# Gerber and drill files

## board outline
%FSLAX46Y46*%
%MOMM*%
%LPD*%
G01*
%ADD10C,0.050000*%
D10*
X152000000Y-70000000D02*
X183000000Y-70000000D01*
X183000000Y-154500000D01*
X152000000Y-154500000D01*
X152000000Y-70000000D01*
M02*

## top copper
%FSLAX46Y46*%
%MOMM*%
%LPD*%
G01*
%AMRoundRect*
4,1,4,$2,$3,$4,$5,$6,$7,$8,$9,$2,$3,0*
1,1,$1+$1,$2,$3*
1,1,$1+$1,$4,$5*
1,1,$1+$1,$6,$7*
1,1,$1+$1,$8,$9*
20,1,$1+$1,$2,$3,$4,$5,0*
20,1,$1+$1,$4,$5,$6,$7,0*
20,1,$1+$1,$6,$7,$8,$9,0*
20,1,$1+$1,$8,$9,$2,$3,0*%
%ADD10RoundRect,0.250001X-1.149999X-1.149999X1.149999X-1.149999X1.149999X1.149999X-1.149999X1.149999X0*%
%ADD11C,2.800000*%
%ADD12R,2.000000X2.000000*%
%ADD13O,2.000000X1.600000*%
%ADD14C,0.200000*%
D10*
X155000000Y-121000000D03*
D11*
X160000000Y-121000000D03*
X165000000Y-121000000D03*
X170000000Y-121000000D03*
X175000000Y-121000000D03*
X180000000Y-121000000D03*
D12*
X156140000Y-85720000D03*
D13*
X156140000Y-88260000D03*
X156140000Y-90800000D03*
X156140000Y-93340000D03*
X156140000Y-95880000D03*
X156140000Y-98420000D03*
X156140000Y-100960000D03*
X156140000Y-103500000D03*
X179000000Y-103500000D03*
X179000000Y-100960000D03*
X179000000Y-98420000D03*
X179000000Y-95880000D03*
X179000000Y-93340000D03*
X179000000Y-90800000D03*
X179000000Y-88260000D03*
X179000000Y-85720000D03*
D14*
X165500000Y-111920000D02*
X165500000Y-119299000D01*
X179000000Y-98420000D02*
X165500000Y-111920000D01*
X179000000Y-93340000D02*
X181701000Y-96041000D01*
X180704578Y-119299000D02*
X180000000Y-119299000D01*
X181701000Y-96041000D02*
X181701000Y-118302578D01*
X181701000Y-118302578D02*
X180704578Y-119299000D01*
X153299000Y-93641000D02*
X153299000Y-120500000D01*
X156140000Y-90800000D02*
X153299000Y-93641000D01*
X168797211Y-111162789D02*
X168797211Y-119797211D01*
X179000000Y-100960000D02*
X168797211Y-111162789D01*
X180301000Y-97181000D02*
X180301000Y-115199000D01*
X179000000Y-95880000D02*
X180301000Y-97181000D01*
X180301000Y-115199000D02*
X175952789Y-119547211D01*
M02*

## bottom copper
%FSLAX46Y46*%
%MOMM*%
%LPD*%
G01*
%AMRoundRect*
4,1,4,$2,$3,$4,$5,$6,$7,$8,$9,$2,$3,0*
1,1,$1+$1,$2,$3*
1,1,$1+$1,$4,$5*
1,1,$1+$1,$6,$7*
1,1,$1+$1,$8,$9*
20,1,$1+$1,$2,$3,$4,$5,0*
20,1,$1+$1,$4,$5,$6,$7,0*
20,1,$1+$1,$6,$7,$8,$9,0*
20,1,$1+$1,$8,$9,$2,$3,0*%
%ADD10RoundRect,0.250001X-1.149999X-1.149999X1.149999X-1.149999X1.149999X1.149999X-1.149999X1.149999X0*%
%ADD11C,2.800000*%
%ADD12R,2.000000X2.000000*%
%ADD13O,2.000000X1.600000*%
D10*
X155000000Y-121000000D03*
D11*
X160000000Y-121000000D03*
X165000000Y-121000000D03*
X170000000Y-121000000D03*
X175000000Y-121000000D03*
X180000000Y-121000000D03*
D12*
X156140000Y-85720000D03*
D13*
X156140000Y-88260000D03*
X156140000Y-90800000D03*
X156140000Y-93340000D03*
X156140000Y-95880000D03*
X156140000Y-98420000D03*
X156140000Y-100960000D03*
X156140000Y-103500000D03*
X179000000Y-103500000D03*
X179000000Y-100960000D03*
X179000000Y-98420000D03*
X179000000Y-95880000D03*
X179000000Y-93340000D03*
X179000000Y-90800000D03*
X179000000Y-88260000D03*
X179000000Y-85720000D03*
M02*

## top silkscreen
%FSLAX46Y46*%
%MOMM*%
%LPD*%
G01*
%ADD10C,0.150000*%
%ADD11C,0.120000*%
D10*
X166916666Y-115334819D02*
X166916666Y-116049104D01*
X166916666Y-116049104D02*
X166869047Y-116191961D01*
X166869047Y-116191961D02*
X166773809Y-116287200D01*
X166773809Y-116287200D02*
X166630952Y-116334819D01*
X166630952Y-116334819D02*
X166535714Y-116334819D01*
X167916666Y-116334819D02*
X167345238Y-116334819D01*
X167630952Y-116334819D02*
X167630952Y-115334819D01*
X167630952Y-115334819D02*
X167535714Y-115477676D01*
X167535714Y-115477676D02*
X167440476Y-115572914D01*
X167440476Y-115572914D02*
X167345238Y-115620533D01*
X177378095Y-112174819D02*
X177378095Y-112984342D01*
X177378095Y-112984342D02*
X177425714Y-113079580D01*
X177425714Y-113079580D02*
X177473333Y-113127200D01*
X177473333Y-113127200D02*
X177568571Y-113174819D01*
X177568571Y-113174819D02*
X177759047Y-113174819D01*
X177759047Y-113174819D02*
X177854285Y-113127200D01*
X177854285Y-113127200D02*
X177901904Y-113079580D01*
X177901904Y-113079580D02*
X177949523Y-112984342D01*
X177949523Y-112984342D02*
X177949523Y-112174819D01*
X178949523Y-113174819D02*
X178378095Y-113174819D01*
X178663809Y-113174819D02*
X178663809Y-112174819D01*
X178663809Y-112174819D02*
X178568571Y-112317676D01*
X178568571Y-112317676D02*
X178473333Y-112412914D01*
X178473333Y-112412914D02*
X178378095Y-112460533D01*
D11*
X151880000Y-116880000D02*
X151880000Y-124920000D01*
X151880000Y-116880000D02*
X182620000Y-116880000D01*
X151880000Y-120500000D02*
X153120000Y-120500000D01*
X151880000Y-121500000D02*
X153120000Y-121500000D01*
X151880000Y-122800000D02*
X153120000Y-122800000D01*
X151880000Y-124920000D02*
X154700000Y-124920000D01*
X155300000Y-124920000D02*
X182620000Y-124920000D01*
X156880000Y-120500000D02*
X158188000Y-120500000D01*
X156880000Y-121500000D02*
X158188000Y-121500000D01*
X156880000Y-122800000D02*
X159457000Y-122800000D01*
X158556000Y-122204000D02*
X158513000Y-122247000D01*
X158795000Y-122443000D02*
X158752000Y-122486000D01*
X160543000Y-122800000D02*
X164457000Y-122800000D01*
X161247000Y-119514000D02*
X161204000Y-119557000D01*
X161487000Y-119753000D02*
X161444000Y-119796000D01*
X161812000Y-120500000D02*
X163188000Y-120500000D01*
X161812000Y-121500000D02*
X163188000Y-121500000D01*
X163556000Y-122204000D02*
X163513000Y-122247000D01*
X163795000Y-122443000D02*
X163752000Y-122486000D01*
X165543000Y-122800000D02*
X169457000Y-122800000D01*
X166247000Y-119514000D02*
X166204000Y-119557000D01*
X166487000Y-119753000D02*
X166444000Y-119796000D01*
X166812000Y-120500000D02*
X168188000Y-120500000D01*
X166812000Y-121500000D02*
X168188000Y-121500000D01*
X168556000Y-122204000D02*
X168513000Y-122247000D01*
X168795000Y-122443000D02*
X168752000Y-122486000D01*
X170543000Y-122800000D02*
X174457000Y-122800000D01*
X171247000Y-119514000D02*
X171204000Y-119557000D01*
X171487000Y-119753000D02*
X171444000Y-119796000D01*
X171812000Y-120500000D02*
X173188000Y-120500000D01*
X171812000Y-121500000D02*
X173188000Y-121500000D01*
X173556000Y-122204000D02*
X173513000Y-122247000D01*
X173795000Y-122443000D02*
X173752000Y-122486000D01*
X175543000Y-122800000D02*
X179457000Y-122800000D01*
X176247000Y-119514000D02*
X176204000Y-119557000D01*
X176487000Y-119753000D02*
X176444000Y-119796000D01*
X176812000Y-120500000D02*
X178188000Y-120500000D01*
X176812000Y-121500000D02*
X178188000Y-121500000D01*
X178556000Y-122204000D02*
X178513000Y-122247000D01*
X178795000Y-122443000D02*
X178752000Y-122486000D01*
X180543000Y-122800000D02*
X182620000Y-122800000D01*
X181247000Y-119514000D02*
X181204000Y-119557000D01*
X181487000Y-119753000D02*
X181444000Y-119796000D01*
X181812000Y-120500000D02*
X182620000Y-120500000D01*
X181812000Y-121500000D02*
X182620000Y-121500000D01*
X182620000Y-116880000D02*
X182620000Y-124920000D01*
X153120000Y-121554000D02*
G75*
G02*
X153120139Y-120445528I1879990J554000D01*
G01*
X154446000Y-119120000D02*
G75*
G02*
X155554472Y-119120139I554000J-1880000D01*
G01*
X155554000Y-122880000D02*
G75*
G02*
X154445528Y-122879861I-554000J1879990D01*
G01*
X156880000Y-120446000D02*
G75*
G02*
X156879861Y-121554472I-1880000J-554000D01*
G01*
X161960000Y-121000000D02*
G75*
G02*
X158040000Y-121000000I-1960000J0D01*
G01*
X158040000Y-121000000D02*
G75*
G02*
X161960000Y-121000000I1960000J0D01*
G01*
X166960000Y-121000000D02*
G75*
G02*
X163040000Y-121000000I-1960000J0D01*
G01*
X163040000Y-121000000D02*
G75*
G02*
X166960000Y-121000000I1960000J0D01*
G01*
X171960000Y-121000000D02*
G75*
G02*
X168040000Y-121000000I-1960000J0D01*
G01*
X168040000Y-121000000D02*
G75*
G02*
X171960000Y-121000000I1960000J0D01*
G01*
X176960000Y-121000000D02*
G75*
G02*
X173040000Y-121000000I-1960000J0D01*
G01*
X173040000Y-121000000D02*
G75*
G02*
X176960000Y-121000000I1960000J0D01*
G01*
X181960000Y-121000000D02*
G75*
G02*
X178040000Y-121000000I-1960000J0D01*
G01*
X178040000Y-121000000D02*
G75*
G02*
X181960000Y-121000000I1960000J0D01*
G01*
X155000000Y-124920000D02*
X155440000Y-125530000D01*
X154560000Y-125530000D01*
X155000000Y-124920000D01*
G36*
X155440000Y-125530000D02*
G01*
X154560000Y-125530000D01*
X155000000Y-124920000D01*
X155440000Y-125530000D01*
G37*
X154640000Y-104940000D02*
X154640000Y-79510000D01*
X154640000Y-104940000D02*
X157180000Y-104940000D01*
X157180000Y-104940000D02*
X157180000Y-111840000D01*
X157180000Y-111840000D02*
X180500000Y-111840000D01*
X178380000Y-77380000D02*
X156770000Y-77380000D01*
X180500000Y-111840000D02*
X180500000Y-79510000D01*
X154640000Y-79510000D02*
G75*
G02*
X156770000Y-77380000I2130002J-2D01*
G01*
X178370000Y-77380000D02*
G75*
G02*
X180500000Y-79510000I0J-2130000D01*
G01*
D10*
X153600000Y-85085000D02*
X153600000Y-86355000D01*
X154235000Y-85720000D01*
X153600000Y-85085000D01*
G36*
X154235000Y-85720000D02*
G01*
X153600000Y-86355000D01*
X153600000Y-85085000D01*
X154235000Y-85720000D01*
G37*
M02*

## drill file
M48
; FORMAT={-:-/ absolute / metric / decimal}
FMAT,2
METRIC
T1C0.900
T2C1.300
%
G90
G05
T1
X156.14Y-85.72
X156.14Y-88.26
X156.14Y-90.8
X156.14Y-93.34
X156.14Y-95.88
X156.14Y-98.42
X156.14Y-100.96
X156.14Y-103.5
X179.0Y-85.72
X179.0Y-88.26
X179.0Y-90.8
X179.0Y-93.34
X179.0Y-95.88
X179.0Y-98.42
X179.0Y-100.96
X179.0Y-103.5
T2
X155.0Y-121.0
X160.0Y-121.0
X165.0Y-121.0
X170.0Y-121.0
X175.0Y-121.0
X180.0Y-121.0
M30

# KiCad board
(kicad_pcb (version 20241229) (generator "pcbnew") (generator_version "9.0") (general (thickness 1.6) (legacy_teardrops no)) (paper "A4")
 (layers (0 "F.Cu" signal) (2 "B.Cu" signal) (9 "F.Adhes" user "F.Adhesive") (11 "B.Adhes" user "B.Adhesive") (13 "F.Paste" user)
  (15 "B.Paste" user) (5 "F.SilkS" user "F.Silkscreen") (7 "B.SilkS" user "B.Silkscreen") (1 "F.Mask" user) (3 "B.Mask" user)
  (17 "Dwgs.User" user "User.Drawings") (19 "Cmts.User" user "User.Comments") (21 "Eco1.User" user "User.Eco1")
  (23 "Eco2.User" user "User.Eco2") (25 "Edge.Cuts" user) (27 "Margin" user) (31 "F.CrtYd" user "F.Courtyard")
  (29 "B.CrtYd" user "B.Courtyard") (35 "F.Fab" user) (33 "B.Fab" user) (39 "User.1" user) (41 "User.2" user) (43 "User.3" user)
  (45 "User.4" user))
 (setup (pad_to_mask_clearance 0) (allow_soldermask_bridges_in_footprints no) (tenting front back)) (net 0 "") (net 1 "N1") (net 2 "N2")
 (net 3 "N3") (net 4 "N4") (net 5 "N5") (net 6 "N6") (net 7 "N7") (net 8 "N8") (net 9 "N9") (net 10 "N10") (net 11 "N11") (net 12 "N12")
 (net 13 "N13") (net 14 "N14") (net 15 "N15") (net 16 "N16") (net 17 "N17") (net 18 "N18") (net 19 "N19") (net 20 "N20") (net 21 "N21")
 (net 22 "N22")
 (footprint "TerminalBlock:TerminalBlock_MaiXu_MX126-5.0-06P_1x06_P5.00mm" (layer "F.Cu") (at 155 121)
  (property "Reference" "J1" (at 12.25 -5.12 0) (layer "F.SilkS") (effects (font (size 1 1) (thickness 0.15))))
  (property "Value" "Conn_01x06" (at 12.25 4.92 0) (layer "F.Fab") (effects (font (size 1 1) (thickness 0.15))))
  (fp_line (start -3.12 -4.12) (end -3.12 3.92) (stroke (width 0.12) (type solid)) (layer "F.SilkS"))
  (fp_line (start -3.12 -4.12) (end 27.62 -4.12) (stroke (width 0.12) (type solid)) (layer "F.SilkS"))
  (fp_line (start -3.12 -0.5) (end -1.88 -0.5) (stroke (width 0.12) (type solid)) (layer "F.SilkS"))
  (fp_line (start -3.12 0.5) (end -1.88 0.5) (stroke (width 0.12) (type solid)) (layer "F.SilkS"))
  (fp_line (start -3.12 1.8) (end -1.88 1.8) (stroke (width 0.12) (type solid)) (layer "F.SilkS"))
  (fp_line (start -3.12 3.92) (end -0.3 3.92) (stroke (width 0.12) (type solid)) (layer "F.SilkS"))
  (fp_line (start 0.3 3.92) (end 27.62 3.92) (stroke (width 0.12) (type solid)) (layer "F.SilkS"))
  (fp_line (start 1.88 -0.5) (end 3.188 -0.5) (stroke (width 0.12) (type solid)) (layer "F.SilkS"))
  (fp_line (start 1.88 0.5) (end 3.188 0.5) (stroke (width 0.12) (type solid)) (layer "F.SilkS"))
  (fp_line (start 1.88 1.8) (end 4.457 1.8) (stroke (width 0.12) (type solid)) (layer "F.SilkS"))
  (fp_line (start 3.556 1.204) (end 3.513 1.247) (stroke (width 0.12) (type solid)) (layer "F.SilkS"))
  (fp_line (start 3.795 1.443) (end 3.752 1.486) (stroke (width 0.12) (type solid)) (layer "F.SilkS"))
  (fp_line (start 5.543 1.8) (end 9.457 1.8) (stroke (width 0.12) (type solid)) (layer "F.SilkS"))
  (fp_line (start 6.247 -1.486) (end 6.204 -1.443) (stroke (width 0.12) (type solid)) (layer "F.SilkS"))
  (fp_line (start 6.487 -1.247) (end 6.444 -1.204) (stroke (width 0.12) (type solid)) (layer "F.SilkS"))
  (fp_line (start 6.812 -0.5) (end 8.188 -0.5) (stroke (width 0.12) (type solid)) (layer "F.SilkS"))
  (fp_line (start 6.812 0.5) (end 8.188 0.5) (stroke (width 0.12) (type solid)) (layer "F.SilkS"))
  (fp_line (start 8.556 1.204) (end 8.513 1.247) (stroke (width 0.12) (type solid)) (layer "F.SilkS"))
  (fp_line (start 8.795 1.443) (end 8.752 1.486) (stroke (width 0.12) (type solid)) (layer "F.SilkS"))
  (fp_line (start 10.543 1.8) (end 14.457 1.8) (stroke (width 0.12) (type solid)) (layer "F.SilkS"))
  (fp_line (start 11.247 -1.486) (end 11.204 -1.443) (stroke (width 0.12) (type solid)) (layer "F.SilkS"))
  (fp_line (start 11.487 -1.247) (end 11.444 -1.204) (stroke (width 0.12) (type solid)) (layer "F.SilkS"))
  (fp_line (start 11.812 -0.5) (end 13.188 -0.5) (stroke (width 0.12) (type solid)) (layer "F.SilkS"))
  (fp_line (start 11.812 0.5) (end 13.188 0.5) (stroke (width 0.12) (type solid)) (layer "F.SilkS"))
  (fp_line (start 13.556 1.204) (end 13.513 1.247) (stroke (width 0.12) (type solid)) (layer "F.SilkS"))
  (fp_line (start 13.795 1.443) (end 13.752 1.486) (stroke (width 0.12) (type solid)) (layer "F.SilkS"))
  (fp_line (start 15.543 1.8) (end 19.457 1.8) (stroke (width 0.12) (type solid)) (layer "F.SilkS"))
  (fp_line (start 16.247 -1.486) (end 16.204 -1.443) (stroke (width 0.12) (type solid)) (layer "F.SilkS"))
  (fp_line (start 16.487 -1.247) (end 16.444 -1.204) (stroke (width 0.12) (type solid)) (layer "F.SilkS"))
  (fp_line (start 16.812 -0.5) (end 18.188 -0.5) (stroke (width 0.12) (type solid)) (layer "F.SilkS"))
  (fp_line (start 16.812 0.5) (end 18.188 0.5) (stroke (width 0.12) (type solid)) (layer "F.SilkS"))
  (fp_line (start 18.556 1.204) (end 18.513 1.247) (stroke (width 0.12) (type solid)) (layer "F.SilkS"))
  (fp_line (start 18.795 1.443) (end 18.752 1.486) (stroke (width 0.12) (type solid)) (layer "F.SilkS"))
  (fp_line (start 20.543 1.8) (end 24.457 1.8) (stroke (width 0.12) (type solid)) (layer "F.SilkS"))
  (fp_line (start 21.247 -1.486) (end 21.204 -1.443) (stroke (width 0.12) (type solid)) (layer "F.SilkS"))
  (fp_line (start 21.487 -1.247) (end 21.444 -1.204) (stroke (width 0.12) (type solid)) (layer "F.SilkS"))
  (fp_line (start 21.812 -0.5) (end 23.188 -0.5) (stroke (width 0.12) (type solid)) (layer "F.SilkS"))
  (fp_line (start 21.812 0.5) (end 23.188 0.5) (stroke (width 0.12) (type solid)) (layer "F.SilkS"))
  (fp_line (start 23.556 1.204) (end 23.513 1.247) (stroke (width 0.12) (type solid)) (layer "F.SilkS"))
  (fp_line (start 23.795 1.443) (end 23.752 1.486) (stroke (width 0.12) (type solid)) (layer "F.SilkS"))
  (fp_line (start 25.543 1.8) (end 27.62 1.8) (stroke (width 0.12) (type solid)) (layer "F.SilkS"))
  (fp_line (start 26.247 -1.486) (end 26.204 -1.443) (stroke (width 0.12) (type solid)) (layer "F.SilkS"))
  (fp_line (start 26.487 -1.247) (end 26.444 -1.204) (stroke (width 0.12) (type solid)) (layer "F.SilkS"))
  (fp_line (start 26.812 -0.5) (end 27.62 -0.5) (stroke (width 0.12) (type solid)) (layer "F.SilkS"))
  (fp_line (start 26.812 0.5) (end 27.62 0.5) (stroke (width 0.12) (type solid)) (layer "F.SilkS"))
  (fp_line (start 27.62 -4.12) (end 27.62 3.92) (stroke (width 0.12) (type solid)) (layer "F.SilkS"))
  (fp_arc (start -1.88 0.554) (mid -1.959928 -0.000246) (end -1.879861 -0.554472) (stroke (width 0.12) (type solid)) (layer "F.SilkS"))
  (fp_arc (start -0.554 -1.88) (mid 0.000246 -1.959928) (end 0.554472 -1.879861) (stroke (width 0.12) (type solid)) (layer "F.SilkS"))
  (fp_arc (start 0.554 1.88) (mid -0.000246 1.959928) (end -0.554472 1.879861) (stroke (width 0.12) (type solid)) (layer "F.SilkS"))
  (fp_arc (start 1.88 -0.554) (mid 1.959928 0.000246) (end 1.879861 0.554472) (stroke (width 0.12) (type solid)) (layer "F.SilkS"))
  (fp_circle (center 5 0) (end 6.96 0) (stroke (width 0.12) (type solid)) (fill no) (layer "F.SilkS"))
  (fp_circle (center 10 0) (end 11.96 0) (stroke (width 0.12) (type solid)) (fill no) (layer "F.SilkS"))
  (fp_circle (center 15 0) (end 16.96 0) (stroke (width 0.12) (type solid)) (fill no) (layer "F.SilkS"))
  (fp_circle (center 20 0) (end 21.96 0) (stroke (width 0.12) (type solid)) (fill no) (layer "F.SilkS"))
  (fp_circle (center 25 0) (end 26.96 0) (stroke (width 0.12) (type solid)) (fill no) (layer "F.SilkS"))
  (fp_poly (pts (xy 0 3.92) (xy 0.44 4.53) (xy -0.44 4.53) (xy 0 3.92)) (stroke (width 0.12) (type solid)) (fill yes) (layer "F.SilkS"))
  (pad "1" thru_hole roundrect (at 0 0) (size 2.8 2.8) (drill 1.3) (layers "*.Cu" "*.Mask") (remove_unused_layers no)
   (roundrect_rratio 0.089286) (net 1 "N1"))
  (pad "2" thru_hole circle (at 5 0) (size 2.8 2.8) (drill 1.3) (layers "*.Cu" "*.Mask") (remove_unused_layers no) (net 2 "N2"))
  (pad "3" thru_hole circle (at 10 0) (size 2.8 2.8) (drill 1.3) (layers "*.Cu" "*.Mask") (remove_unused_layers no) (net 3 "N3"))
  (pad "4" thru_hole circle (at 15 0) (size 2.8 2.8) (drill 1.3) (layers "*.Cu" "*.Mask") (remove_unused_layers no) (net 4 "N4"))
  (pad "5" thru_hole circle (at 20 0) (size 2.8 2.8) (drill 1.3) (layers "*.Cu" "*.Mask") (remove_unused_layers no) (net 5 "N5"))
  (pad "6" thru_hole circle (at 25 0) (size 2.8 2.8) (drill 1.3) (layers "*.Cu" "*.Mask") (remove_unused_layers no) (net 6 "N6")))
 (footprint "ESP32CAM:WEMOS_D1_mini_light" (layer "F.Cu") (at 156.14 85.72)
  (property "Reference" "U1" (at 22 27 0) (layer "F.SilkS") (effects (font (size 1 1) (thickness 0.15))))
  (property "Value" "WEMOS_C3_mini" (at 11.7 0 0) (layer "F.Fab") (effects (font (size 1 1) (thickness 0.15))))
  (fp_line (start -1.5 19.22) (end -1.5 -6.21) (stroke (width 0.12) (type solid)) (layer "F.SilkS"))
  (fp_line (start -1.5 19.22) (end 1.04 19.22) (stroke (width 0.12) (type solid)) (layer "F.SilkS"))
  (fp_line (start 1.04 19.22) (end 1.04 26.12) (stroke (width 0.12) (type solid)) (layer "F.SilkS"))
  (fp_line (start 1.04 26.12) (end 24.36 26.12) (stroke (width 0.12) (type solid)) (layer "F.SilkS"))
  (fp_line (start 22.24 -8.34) (end 0.63 -8.34) (stroke (width 0.12) (type solid)) (layer "F.SilkS"))
  (fp_line (start 24.36 26.12) (end 24.36 -6.21) (stroke (width 0.12) (type solid)) (layer "F.SilkS"))
  (fp_arc (start -1.5 -6.21) (mid -0.876137 -7.716137) (end 0.63 -8.34) (stroke (width 0.12) (type solid)) (layer "F.SilkS"))
  (fp_arc (start 22.23 -8.34) (mid 23.736137 -7.716137) (end 24.36 -6.21) (stroke (width 0.12) (type solid)) (layer "F.SilkS"))
  (fp_poly (pts (xy -2.54 -0.635) (xy -2.54 0.635) (xy -1.905 0)) (stroke (width 0.15) (type solid)) (fill yes) (layer "F.SilkS"))
  (pad "1" thru_hole rect (at 0 0) (size 2 2) (drill 0.9) (layers "*.Cu" "*.Mask") (remove_unused_layers no) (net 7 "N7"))
  (pad "2" thru_hole oval (at 0 2.54) (size 2 1.6) (drill 0.9) (layers "*.Cu" "*.Mask") (remove_unused_layers no) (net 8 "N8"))
  (pad "3" thru_hole oval (at 0 5.08) (size 2 1.6) (drill 0.9) (layers "*.Cu" "*.Mask") (remove_unused_layers no) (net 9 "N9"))
  (pad "4" thru_hole oval (at 0 7.62) (size 2 1.6) (drill 0.9) (layers "*.Cu" "*.Mask") (remove_unused_layers no) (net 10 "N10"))
  (pad "5" thru_hole oval (at 0 10.16) (size 2 1.6) (drill 0.9) (layers "*.Cu" "*.Mask") (remove_unused_layers no) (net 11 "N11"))
  (pad "6" thru_hole oval (at 0 12.7) (size 2 1.6) (drill 0.9) (layers "*.Cu" "*.Mask") (remove_unused_layers no) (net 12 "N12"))
  (pad "7" thru_hole oval (at 0 15.24) (size 2 1.6) (drill 0.9) (layers "*.Cu" "*.Mask") (remove_unused_layers no) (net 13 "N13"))
  (pad "8" thru_hole oval (at 0 17.78) (size 2 1.6) (drill 0.9) (layers "*.Cu" "*.Mask") (remove_unused_layers no) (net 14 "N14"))
  (pad "9" thru_hole oval (at 22.86 17.78) (size 2 1.6) (drill 0.9) (layers "*.Cu" "*.Mask") (remove_unused_layers no) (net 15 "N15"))
  (pad "10" thru_hole oval (at 22.86 15.24) (size 2 1.6) (drill 0.9) (layers "*.Cu" "*.Mask") (remove_unused_layers no) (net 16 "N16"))
  (pad "11" thru_hole oval (at 22.86 12.7) (size 2 1.6) (drill 0.9) (layers "*.Cu" "*.Mask") (remove_unused_layers no) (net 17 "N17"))
  (pad "12" thru_hole oval (at 22.86 10.16) (size 2 1.6) (drill 0.9) (layers "*.Cu" "*.Mask") (remove_unused_layers no) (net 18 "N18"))
  (pad "13" thru_hole oval (at 22.86 7.62) (size 2 1.6) (drill 0.9) (layers "*.Cu" "*.Mask") (remove_unused_layers no) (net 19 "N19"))
  (pad "14" thru_hole oval (at 22.86 5.08) (size 2 1.6) (drill 0.9) (layers "*.Cu" "*.Mask") (remove_unused_layers no) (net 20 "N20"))
  (pad "15" thru_hole oval (at 22.86 2.54) (size 2 1.6) (drill 0.9) (layers "*.Cu" "*.Mask") (remove_unused_layers no) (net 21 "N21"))
  (pad "16" thru_hole oval (at 22.86 0) (size 2 1.6) (drill 0.9) (layers "*.Cu" "*.Mask") (remove_unused_layers no) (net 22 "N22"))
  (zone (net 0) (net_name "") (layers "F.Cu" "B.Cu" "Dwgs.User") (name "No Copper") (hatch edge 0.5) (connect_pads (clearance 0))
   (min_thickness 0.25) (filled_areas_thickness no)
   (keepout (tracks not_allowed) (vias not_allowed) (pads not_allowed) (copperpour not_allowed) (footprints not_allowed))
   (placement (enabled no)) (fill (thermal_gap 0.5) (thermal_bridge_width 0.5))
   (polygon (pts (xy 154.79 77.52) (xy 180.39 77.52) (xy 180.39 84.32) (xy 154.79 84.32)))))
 (gr_rect (start 152 70) (end 183 154.5) (stroke (width 0.05) (type default)) (fill no) (layer "Edge.Cuts"))
 (segment (start 165.5 111.92) (end 165.5 119.299) (width 0.2) (layer "F.Cu") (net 17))
 (segment (start 179 98.42) (end 165.5 111.92) (width 0.2) (layer "F.Cu") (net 17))
 (segment (start 179 93.34) (end 181.701 96.041) (width 0.2) (layer "F.Cu") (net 19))
 (segment (start 180.704578 119.299) (end 180 119.299) (width 0.2) (layer "F.Cu") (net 19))
 (segment (start 181.701 96.041) (end 181.701 118.302578) (width 0.2) (layer "F.Cu") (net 19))
 (segment (start 181.701 118.302578) (end 180.704578 119.299) (width 0.2) (layer "F.Cu") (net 19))
 (segment (start 153.299 93.641) (end 153.299 120.5) (width 0.2) (layer "F.Cu") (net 9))
 (segment (start 156.14 90.8) (end 153.299 93.641) (width 0.2) (layer "F.Cu") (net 9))
 (segment (start 168.797211 111.162789) (end 168.797211 119.797211) (width 0.2) (layer "F.Cu") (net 16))
 (segment (start 179 100.96) (end 168.797211 111.162789) (width 0.2) (layer "F.Cu") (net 16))
 (segment (start 180.301 97.181) (end 180.301 115.199) (width 0.2) (layer "F.Cu") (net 18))
 (segment (start 179 95.88) (end 180.301 97.181) (width 0.2) (layer "F.Cu") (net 18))
 (segment (start 180.301 115.199) (end 175.952789 119.547211) (width 0.2) (layer "F.Cu") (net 18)))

